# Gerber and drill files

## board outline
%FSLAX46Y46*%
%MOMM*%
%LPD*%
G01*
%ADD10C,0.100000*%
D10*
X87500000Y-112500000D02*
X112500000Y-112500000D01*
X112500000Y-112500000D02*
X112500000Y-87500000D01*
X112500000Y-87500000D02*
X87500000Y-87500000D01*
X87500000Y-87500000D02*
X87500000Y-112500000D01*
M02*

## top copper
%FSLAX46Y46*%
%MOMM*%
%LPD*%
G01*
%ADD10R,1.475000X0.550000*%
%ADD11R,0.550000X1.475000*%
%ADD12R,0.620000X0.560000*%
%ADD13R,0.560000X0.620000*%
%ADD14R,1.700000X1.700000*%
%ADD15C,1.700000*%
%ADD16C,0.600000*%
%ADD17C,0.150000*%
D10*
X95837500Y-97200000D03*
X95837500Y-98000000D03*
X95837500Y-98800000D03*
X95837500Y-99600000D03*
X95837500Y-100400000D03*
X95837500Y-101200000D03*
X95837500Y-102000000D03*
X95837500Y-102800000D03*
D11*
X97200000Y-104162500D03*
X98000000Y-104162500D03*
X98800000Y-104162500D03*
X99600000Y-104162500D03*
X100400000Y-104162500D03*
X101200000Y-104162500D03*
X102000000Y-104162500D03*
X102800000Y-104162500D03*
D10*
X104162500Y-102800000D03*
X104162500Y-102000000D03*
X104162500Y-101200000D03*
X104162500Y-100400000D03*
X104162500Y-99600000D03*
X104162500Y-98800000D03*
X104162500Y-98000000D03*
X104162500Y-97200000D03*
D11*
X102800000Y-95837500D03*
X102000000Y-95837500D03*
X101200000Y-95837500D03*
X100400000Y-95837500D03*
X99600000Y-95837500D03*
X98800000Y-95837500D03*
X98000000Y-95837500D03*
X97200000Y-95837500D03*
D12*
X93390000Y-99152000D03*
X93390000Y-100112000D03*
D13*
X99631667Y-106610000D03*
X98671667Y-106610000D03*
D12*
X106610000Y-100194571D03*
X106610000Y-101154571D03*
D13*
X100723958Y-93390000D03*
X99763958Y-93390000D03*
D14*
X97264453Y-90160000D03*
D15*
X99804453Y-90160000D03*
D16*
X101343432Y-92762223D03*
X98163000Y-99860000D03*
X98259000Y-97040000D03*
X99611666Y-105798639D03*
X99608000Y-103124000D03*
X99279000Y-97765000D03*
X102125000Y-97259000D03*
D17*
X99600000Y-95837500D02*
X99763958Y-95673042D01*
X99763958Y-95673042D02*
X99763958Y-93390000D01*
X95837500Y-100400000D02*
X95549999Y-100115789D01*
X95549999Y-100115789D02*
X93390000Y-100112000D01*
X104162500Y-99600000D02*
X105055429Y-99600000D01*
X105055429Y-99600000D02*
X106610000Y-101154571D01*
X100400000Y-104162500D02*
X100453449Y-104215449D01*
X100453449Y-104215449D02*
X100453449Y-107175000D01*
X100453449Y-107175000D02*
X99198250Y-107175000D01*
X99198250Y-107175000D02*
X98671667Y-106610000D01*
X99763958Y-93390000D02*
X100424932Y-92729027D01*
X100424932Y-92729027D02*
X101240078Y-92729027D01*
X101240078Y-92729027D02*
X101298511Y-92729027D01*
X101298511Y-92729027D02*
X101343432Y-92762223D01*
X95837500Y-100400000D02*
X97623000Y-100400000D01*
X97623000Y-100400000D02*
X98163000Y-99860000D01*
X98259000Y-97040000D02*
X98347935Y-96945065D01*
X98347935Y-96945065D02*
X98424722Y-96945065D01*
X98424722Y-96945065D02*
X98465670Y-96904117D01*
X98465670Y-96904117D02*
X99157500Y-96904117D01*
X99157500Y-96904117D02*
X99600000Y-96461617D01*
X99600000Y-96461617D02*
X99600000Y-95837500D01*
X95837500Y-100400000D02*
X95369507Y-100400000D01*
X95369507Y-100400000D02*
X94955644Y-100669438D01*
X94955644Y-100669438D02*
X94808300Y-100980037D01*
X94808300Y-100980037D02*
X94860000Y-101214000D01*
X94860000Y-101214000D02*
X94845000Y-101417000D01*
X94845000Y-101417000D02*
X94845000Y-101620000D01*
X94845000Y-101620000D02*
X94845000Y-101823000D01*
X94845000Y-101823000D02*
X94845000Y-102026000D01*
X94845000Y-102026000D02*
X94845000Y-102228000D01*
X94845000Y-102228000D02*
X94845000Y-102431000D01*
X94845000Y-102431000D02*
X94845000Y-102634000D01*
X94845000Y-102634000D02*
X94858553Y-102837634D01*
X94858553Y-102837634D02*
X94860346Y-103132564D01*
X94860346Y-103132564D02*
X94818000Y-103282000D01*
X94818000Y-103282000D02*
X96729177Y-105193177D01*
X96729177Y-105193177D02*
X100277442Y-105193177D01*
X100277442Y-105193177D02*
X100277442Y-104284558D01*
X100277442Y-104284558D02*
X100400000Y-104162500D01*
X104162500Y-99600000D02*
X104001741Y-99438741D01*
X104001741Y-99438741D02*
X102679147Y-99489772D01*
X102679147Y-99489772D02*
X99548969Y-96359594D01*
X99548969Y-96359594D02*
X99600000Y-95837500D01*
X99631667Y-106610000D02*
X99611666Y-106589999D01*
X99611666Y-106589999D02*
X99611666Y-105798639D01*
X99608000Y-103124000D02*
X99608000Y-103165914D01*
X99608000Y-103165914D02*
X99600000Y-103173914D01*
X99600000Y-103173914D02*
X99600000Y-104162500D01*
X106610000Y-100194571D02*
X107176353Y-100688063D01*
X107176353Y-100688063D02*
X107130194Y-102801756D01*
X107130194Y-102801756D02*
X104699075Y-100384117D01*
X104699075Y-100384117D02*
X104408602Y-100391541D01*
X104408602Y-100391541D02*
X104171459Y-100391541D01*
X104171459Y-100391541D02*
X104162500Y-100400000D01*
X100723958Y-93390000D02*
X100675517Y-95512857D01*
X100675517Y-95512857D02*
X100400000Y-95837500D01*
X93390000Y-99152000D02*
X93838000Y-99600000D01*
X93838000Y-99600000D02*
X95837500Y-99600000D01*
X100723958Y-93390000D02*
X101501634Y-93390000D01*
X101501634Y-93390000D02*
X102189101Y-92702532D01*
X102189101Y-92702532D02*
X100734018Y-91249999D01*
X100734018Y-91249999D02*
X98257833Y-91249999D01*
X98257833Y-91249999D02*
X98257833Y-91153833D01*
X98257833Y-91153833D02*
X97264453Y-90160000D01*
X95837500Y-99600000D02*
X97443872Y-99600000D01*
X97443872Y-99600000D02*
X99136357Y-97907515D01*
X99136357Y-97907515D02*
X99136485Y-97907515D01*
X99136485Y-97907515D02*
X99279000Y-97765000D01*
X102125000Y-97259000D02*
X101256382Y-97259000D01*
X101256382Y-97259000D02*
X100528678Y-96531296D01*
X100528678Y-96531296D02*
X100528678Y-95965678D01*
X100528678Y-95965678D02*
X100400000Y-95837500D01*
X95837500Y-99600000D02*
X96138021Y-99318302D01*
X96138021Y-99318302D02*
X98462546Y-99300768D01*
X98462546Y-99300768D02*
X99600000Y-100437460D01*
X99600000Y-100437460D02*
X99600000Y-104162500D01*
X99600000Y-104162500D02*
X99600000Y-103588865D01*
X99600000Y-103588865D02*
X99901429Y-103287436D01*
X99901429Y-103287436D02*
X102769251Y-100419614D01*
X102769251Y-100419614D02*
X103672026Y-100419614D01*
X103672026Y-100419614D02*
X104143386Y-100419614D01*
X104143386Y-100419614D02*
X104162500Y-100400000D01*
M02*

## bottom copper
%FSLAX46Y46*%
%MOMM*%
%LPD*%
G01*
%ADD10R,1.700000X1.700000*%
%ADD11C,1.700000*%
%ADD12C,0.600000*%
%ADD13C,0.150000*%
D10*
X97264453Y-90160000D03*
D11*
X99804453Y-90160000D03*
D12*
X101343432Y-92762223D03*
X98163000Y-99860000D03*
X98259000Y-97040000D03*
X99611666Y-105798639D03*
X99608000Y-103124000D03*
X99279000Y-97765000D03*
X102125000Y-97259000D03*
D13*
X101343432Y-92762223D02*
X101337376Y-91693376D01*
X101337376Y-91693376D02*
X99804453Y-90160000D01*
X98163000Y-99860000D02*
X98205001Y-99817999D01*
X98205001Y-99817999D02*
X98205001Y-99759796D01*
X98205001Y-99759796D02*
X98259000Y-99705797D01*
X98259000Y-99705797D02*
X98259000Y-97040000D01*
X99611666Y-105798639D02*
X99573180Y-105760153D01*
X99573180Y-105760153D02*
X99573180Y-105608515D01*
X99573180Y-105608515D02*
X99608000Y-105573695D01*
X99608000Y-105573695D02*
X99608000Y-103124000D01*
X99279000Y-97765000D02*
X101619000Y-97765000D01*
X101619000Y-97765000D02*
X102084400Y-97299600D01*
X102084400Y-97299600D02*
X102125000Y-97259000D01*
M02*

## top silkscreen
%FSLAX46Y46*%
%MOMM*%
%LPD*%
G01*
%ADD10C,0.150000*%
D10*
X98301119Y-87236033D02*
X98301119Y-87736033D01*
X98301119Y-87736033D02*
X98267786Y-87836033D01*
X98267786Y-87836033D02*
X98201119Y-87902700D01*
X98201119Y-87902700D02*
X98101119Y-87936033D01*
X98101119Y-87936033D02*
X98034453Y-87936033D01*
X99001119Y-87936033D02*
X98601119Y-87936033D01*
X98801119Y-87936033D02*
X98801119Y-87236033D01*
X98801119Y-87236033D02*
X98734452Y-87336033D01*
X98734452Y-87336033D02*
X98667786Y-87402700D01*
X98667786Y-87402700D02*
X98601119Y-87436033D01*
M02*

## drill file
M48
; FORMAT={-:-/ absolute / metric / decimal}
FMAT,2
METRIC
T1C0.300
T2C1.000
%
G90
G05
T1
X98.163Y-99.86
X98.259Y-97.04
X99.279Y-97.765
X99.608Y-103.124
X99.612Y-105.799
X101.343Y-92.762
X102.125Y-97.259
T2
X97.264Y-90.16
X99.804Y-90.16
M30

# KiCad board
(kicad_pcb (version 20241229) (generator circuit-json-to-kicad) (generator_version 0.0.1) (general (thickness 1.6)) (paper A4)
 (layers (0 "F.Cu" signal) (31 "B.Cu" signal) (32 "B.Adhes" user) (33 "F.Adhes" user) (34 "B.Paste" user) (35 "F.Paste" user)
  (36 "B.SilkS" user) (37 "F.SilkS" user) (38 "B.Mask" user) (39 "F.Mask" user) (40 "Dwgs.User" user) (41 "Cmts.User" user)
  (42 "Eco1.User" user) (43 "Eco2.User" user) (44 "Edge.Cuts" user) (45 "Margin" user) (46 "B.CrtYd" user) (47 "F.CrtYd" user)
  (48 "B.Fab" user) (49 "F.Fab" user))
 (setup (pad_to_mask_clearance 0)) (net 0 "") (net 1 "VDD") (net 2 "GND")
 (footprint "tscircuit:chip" (layer F.Cu) (at 100 100 0)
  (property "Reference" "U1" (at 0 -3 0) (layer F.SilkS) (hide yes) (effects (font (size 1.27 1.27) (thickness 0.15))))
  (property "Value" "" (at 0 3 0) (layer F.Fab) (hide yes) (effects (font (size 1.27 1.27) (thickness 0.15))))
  (pad "1" smd rect (at -4.1625 -2.8 0) (size 1.475 0.55) (layers F.Cu F.Mask))
  (pad "2" smd rect (at -4.1625 -2 0) (size 1.475 0.55) (layers F.Cu F.Mask))
  (pad "3" smd rect (at -4.1625 -1.2 0) (size 1.475 0.55) (layers F.Cu F.Mask))
  (pad "4" smd rect (at -4.1625 -0.4 0) (size 1.475 0.55) (layers F.Cu F.Mask) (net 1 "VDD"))
  (pad "5" smd rect (at -4.1625 0.4 0) (size 1.475 0.55) (layers F.Cu F.Mask) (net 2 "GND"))
  (pad "6" smd rect (at -4.1625 1.2 0) (size 1.475 0.55) (layers F.Cu F.Mask))
  (pad "7" smd rect (at -4.1625 2 0) (size 1.475 0.55) (layers F.Cu F.Mask))
  (pad "8" smd rect (at -4.1625 2.8 0) (size 1.475 0.55) (layers F.Cu F.Mask))
  (pad "9" smd rect (at -2.8 4.1625 0) (size 0.55 1.475) (layers F.Cu F.Mask))
  (pad "10" smd rect (at -2 4.1625 0) (size 0.55 1.475) (layers F.Cu F.Mask))
  (pad "11" smd rect (at -1.2 4.1625 0) (size 0.55 1.475) (layers F.Cu F.Mask))
  (pad "12" smd rect (at -0.4 4.1625 0) (size 0.55 1.475) (layers F.Cu F.Mask) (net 1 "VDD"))
  (pad "13" smd rect (at 0.4 4.1625 0) (size 0.55 1.475) (layers F.Cu F.Mask) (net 2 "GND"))
  (pad "14" smd rect (at 1.2 4.1625 0) (size 0.55 1.475) (layers F.Cu F.Mask))
  (pad "15" smd rect (at 2 4.1625 0) (size 0.55 1.475) (layers F.Cu F.Mask))
  (pad "16" smd rect (at 2.8 4.1625 0) (size 0.55 1.475) (layers F.Cu F.Mask))
  (pad "17" smd rect (at 4.1625 2.8 0) (size 1.475 0.55) (layers F.Cu F.Mask))
  (pad "18" smd rect (at 4.1625 2 0) (size 1.475 0.55) (layers F.Cu F.Mask))
  (pad "19" smd rect (at 4.1625 1.2 0) (size 1.475 0.55) (layers F.Cu F.Mask))
  (pad "20" smd rect (at 4.1625 0.4 0) (size 1.475 0.55) (layers F.Cu F.Mask) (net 1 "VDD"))
  (pad "21" smd rect (at 4.1625 -0.4 0) (size 1.475 0.55) (layers F.Cu F.Mask) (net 2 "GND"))
  (pad "22" smd rect (at 4.1625 -1.2 0) (size 1.475 0.55) (layers F.Cu F.Mask))
  (pad "23" smd rect (at 4.1625 -2 0) (size 1.475 0.55) (layers F.Cu F.Mask))
  (pad "24" smd rect (at 4.1625 -2.8 0) (size 1.475 0.55) (layers F.Cu F.Mask))
  (pad "25" smd rect (at 2.8 -4.1625 0) (size 0.55 1.475) (layers F.Cu F.Mask))
  (pad "26" smd rect (at 2 -4.1625 0) (size 0.55 1.475) (layers F.Cu F.Mask))
  (pad "27" smd rect (at 1.2 -4.1625 0) (size 0.55 1.475) (layers F.Cu F.Mask))
  (pad "28" smd rect (at 0.4 -4.1625 0) (size 0.55 1.475) (layers F.Cu F.Mask) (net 1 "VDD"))
  (pad "29" smd rect (at -0.4 -4.1625 0) (size 0.55 1.475) (layers F.Cu F.Mask) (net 2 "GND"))
  (pad "30" smd rect (at -1.2 -4.1625 0) (size 0.55 1.475) (layers F.Cu F.Mask))
  (pad "31" smd rect (at -2 -4.1625 0) (size 0.55 1.475) (layers F.Cu F.Mask))
  (pad "32" smd rect (at -2.8 -4.1625 0) (size 0.55 1.475) (layers F.Cu F.Mask))
  (pad "" smd rect (at -4.1625 -2.8 0) (size 1.0325 0.385) (layers F.Paste))
  (pad "" smd rect (at -4.1625 -2 0) (size 1.0325 0.385) (layers F.Paste))
  (pad "" smd rect (at -4.1625 -1.2 0) (size 1.0325 0.385) (layers F.Paste))
  (pad "" smd rect (at -4.1625 -0.4 0) (size 1.0325 0.385) (layers F.Paste))
  (pad "" smd rect (at -4.1625 0.4 0) (size 1.0325 0.385) (layers F.Paste))
  (pad "" smd rect (at -4.1625 1.2 0) (size 1.0325 0.385) (layers F.Paste))
  (pad "" smd rect (at -4.1625 2 0) (size 1.0325 0.385) (layers F.Paste))
  (pad "" smd rect (at -4.1625 2.8 0) (size 1.0325 0.385) (layers F.Paste))
  (pad "" smd rect (at -2.8 4.1625 0) (size 0.385 1.0325) (layers F.Paste))
  (pad "" smd rect (at -2 4.1625 0) (size 0.385 1.0325) (layers F.Paste))
  (pad "" smd rect (at -1.2 4.1625 0) (size 0.385 1.0325) (layers F.Paste))
  (pad "" smd rect (at -0.4 4.1625 0) (size 0.385 1.0325) (layers F.Paste))
  (pad "" smd rect (at 0.4 4.1625 0) (size 0.385 1.0325) (layers F.Paste))
  (pad "" smd rect (at 1.2 4.1625 0) (size 0.385 1.0325) (layers F.Paste))
  (pad "" smd rect (at 2 4.1625 0) (size 0.385 1.0325) (layers F.Paste))
  (pad "" smd rect (at 2.8 4.1625 0) (size 0.385 1.0325) (layers F.Paste))
  (pad "" smd rect (at 4.1625 2.8 0) (size 1.0325 0.385) (layers F.Paste))
  (pad "" smd rect (at 4.1625 2 0) (size 1.0325 0.385) (layers F.Paste))
  (pad "" smd rect (at 4.1625 1.2 0) (size 1.0325 0.385) (layers F.Paste))
  (pad "" smd rect (at 4.1625 0.4 0) (size 1.0325 0.385) (layers F.Paste))
  (pad "" smd rect (at 4.1625 -0.4 0) (size 1.0325 0.385) (layers F.Paste))
  (pad "" smd rect (at 4.1625 -1.2 0) (size 1.0325 0.385) (layers F.Paste))
  (pad "" smd rect (at 4.1625 -2 0) (size 1.0325 0.385) (layers F.Paste))
  (pad "" smd rect (at 4.1625 -2.8 0) (size 1.0325 0.385) (layers F.Paste))
  (pad "" smd rect (at 2.8 -4.1625 0) (size 0.385 1.0325) (layers F.Paste))
  (pad "" smd rect (at 2 -4.1625 0) (size 0.385 1.0325) (layers F.Paste))
  (pad "" smd rect (at 1.2 -4.1625 0) (size 0.385 1.0325) (layers F.Paste))
  (pad "" smd rect (at 0.4 -4.1625 0) (size 0.385 1.0325) (layers F.Paste))
  (pad "" smd rect (at -0.4 -4.1625 0) (size 0.385 1.0325) (layers F.Paste))
  (pad "" smd rect (at -1.2 -4.1625 0) (size 0.385 1.0325) (layers F.Paste))
  (pad "" smd rect (at -2 -4.1625 0) (size 0.385 1.0325) (layers F.Paste))
  (pad "" smd rect (at -2.8 -4.1625 0) (size 0.385 1.0325) (layers F.Paste)))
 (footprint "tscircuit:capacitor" (layer F.Cu) (at 93.39 99.632 -90.00000000000001)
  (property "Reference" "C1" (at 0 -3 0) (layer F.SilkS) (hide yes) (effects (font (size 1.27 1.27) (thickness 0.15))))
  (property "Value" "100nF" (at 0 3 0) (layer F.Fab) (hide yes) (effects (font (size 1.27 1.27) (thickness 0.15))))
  (pad "1" smd rect (at -0.48 0 0) (size 0.62 0.56) (layers F.Cu F.Mask) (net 1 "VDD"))
  (pad "2" smd rect (at 0.48 0 0) (size 0.62 0.56) (layers F.Cu F.Mask) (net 2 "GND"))
  (pad "" smd rect (at -0.48 0 0) (size 0.434 0.392) (layers F.Paste))
  (pad "" smd rect (at 0.48 0 0) (size 0.434 0.392) (layers F.Paste)))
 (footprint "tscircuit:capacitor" (layer F.Cu) (at 99.15166666666667 106.61 180)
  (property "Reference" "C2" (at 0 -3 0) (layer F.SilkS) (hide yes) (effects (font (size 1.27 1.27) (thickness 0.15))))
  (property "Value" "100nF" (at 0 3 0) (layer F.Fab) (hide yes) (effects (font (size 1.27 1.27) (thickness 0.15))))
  (pad "1" smd rect (at -0.48000000000000004 0 0) (size 0.56 0.62) (layers F.Cu F.Mask) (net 1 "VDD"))
  (pad "2" smd rect (at 0.47999999999999987 0 0) (size 0.56 0.62) (layers F.Cu F.Mask) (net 2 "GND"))
  (pad "" smd rect (at -0.48000000000000004 0 0) (size 0.392 0.434) (layers F.Paste))
  (pad "" smd rect (at 0.47999999999999987 0 0) (size 0.392 0.434) (layers F.Paste)))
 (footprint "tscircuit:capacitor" (layer F.Cu) (at 106.61 100.67457142857143 -90.00000000000001)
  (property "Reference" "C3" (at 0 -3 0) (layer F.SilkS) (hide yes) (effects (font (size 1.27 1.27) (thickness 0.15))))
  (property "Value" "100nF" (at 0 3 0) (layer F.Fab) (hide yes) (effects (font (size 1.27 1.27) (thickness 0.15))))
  (pad "1" smd rect (at -0.48 0 0) (size 0.62 0.56) (layers F.Cu F.Mask) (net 1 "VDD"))
  (pad "2" smd rect (at 0.4800000000000001 0 0) (size 0.62 0.56) (layers F.Cu F.Mask) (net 2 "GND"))
  (pad "" smd rect (at -0.48 0 0) (size 0.434 0.392) (layers F.Paste))
  (pad "" smd rect (at 0.4800000000000001 0 0) (size 0.434 0.392) (layers F.Paste)))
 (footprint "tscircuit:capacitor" (layer F.Cu) (at 100.24395833333334 93.39 180)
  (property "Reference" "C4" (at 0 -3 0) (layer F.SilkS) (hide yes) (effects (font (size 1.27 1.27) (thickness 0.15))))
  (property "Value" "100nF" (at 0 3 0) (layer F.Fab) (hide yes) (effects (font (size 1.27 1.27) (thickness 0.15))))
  (pad "1" smd rect (at -0.48 0 0) (size 0.56 0.62) (layers F.Cu F.Mask) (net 1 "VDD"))
  (pad "2" smd rect (at 0.48 0 0) (size 0.56 0.62) (layers F.Cu F.Mask) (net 2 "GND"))
  (pad "" smd rect (at -0.48 0 0) (size 0.392 0.434) (layers F.Paste))
  (pad "" smd rect (at 0.48 0 0) (size 0.392 0.434) (layers F.Paste)))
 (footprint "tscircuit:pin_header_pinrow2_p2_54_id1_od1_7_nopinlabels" (layer F.Cu) (at 98.534453125 90.16 0)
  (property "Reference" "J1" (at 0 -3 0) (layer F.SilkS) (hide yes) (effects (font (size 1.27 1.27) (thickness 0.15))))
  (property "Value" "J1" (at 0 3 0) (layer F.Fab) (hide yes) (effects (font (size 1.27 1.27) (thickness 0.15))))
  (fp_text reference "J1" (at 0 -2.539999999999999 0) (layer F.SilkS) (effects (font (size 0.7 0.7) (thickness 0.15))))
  (pad "1" thru_hole rect (at -1.27 0 0) (size 1.7 1.7) (drill 1) (layers *.Cu *.Mask) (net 1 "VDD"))
  (pad "2" thru_hole circle (at 1.27 0 0) (size 1.7 1.7) (drill 1) (layers *.Cu *.Mask) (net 2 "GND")))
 (segment (start 99.6 95.8375) (end 99.76395833333333 95.67304166666666) (width 0.15) (layer F.Cu) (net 2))
 (segment (start 99.76395833333333 95.67304166666666) (end 99.76395833333333 93.39) (width 0.15) (layer F.Cu) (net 2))
 (segment (start 95.8375 100.4) (end 95.54999882570709 100.11578913637184) (width 0.15) (layer F.Cu) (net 2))
 (segment (start 95.54999882570709 100.11578913637184) (end 93.39 100.112) (width 0.15) (layer F.Cu) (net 2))
 (segment (start 104.1625 99.6) (end 105.05542857142856 99.6) (width 0.15) (layer F.Cu) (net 2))
 (segment (start 105.05542857142856 99.6) (end 106.61 101.15457142857143) (width 0.15) (layer F.Cu) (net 2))
 (segment (start 100.4 104.1625) (end 100.45344876131234 104.21544876131235) (width 0.15) (layer F.Cu) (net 2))
 (segment (start 100.45344876131234 104.21544876131235) (end 100.45344876131234 107.175) (width 0.15) (layer F.Cu) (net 2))
 (segment (start 100.45344876131234 107.175) (end 99.19824993292859 107.175) (width 0.15) (layer F.Cu) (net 2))
 (segment (start 99.19824993292859 107.175) (end 98.67166666666667 106.61) (width 0.15) (layer F.Cu) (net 2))
 (segment (start 99.76395833333333 93.39) (end 100.42493155843435 92.72902677489898) (width 0.15) (layer F.Cu) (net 2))
 (segment (start 100.42493155843435 92.72902677489898) (end 101.24007779189273 92.72902677489898) (width 0.15) (layer F.Cu) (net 2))
 (segment (start 101.24007779189273 92.72902677489898) (end 101.2985105056803 92.72902677489898) (width 0.15) (layer F.Cu) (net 2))
 (segment (start 101.2985105056803 92.72902677489898) (end 101.34343219516313 92.76222256666912) (width 0.15) (layer F.Cu) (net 2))
 (segment (start 101.34343219516313 92.76222256666912) (end 101.33737570534065 91.69337570534066) (width 0.15) (layer B.Cu) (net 2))
 (segment (start 101.33737570534065 91.69337570534066) (end 99.804453125 90.16) (width 0.15) (layer B.Cu) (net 2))
 (segment (start 95.8375 100.4) (end 97.623 100.4) (width 0.15) (layer F.Cu) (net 2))
 (segment (start 97.623 100.4) (end 98.163 99.86) (width 0.15) (layer F.Cu) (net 2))
 (segment (start 98.163 99.86) (end 98.20500076413374 99.81799923586625) (width 0.15) (layer B.Cu) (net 2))
 (segment (start 98.20500076413374 99.81799923586625) (end 98.20500076413374 99.75979623298763) (width 0.15) (layer B.Cu) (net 2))
 (segment (start 98.20500076413374 99.75979623298763) (end 98.259 99.70579699712138) (width 0.15) (layer B.Cu) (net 2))
 (segment (start 98.259 99.70579699712138) (end 98.259 97.04) (width 0.15) (layer B.Cu) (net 2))
 (segment (start 98.259 97.04) (end 98.34793469358411 96.9450653064159) (width 0.15) (layer F.Cu) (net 2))
 (segment (start 98.34793469358411 96.9450653064159) (end 98.4247223865256 96.9450653064159) (width 0.15) (layer F.Cu) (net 2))
 (segment (start 98.4247223865256 96.9450653064159) (end 98.46567033995531 96.90411735298619) (width 0.15) (layer F.Cu) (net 2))
 (segment (start 98.46567033995531 96.90411735298619) (end 99.15749956172179 96.90411735298619) (width 0.15) (layer F.Cu) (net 2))
 (segment (start 99.15749956172179 96.90411735298619) (end 99.6 96.46161691470799) (width 0.15) (layer F.Cu) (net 2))
 (segment (start 99.6 96.46161691470799) (end 99.6 95.8375) (width 0.15) (layer F.Cu) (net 2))
 (segment (start 95.8375 100.4) (end 95.36950657616131 100.4) (width 0.15) (layer F.Cu) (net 2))
 (segment (start 95.36950657616131 100.4) (end 94.95564404651859 100.66943775485414) (width 0.15) (layer F.Cu) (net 2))
 (segment (start 94.95564404651859 100.66943775485414) (end 94.80829993462471 100.98003654561826) (width 0.15) (layer F.Cu) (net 2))
 (segment (start 94.80829993462471 100.98003654561826) (end 94.86 101.214) (width 0.15) (layer F.Cu) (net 2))
 (segment (start 94.86 101.214) (end 94.845 101.417) (width 0.15) (layer F.Cu) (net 2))
 (segment (start 94.845 101.417) (end 94.845 101.62) (width 0.15) (layer F.Cu) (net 2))
 (segment (start 94.845 101.62) (end 94.845 101.823) (width 0.15) (layer F.Cu) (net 2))
 (segment (start 94.845 101.823) (end 94.845 102.026) (width 0.15) (layer F.Cu) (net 2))
 (segment (start 94.845 102.026) (end 94.845 102.228) (width 0.15) (layer F.Cu) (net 2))
 (segment (start 94.845 102.228) (end 94.845 102.431) (width 0.15) (layer F.Cu) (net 2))
 (segment (start 94.845 102.431) (end 94.845 102.634) (width 0.15) (layer F.Cu) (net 2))
 (segment (start 94.845 102.634) (end 94.85855329042725 102.83763390606946) (width 0.15) (layer F.Cu) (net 2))
 (segment (start 94.85855329042725 102.83763390606946) (end 94.86034600494294 103.1325643967498) (width 0.15) (layer F.Cu) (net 2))
 (segment (start 94.86034600494294 103.1325643967498) (end 94.818 103.282) (width 0.15) (layer F.Cu) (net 2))
 (segment (start 94.818 103.282) (end 96.72917663282733 105.19317663282735) (width 0.15) (layer F.Cu) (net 2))
 (segment (start 96.72917663282733 105.19317663282735) (end 100.27744164139212 105.19317663282735) (width 0.15) (layer F.Cu) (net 2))
 (segment (start 100.27744164139212 105.19317663282735) (end 100.27744164139212 104.28455835860788) (width 0.15) (layer F.Cu) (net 2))
 (segment (start 100.27744164139212 104.28455835860788) (end 100.4 104.1625) (width 0.15) (layer F.Cu) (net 2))
 (segment (start 104.1625 99.6) (end 104.00174073680326 99.43874073680325) (width 0.15) (layer F.Cu) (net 2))
 (segment (start 104.00174073680326 99.43874073680325) (end 102.67914711390605 99.4897715723112) (width 0.15) (layer F.Cu) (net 2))
 (segment (start 102.67914711390605 99.4897715723112) (end 99.54896916449205 96.3595936228972) (width 0.15) (layer F.Cu) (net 2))
 (segment (start 99.54896916449205 96.3595936228972) (end 99.6 95.8375) (width 0.15) (layer F.Cu) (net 2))
 (segment (start 99.63166666666666 106.61) (end 99.61166566666667 106.589999) (width 0.15) (layer F.Cu) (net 1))
 (segment (start 99.61166566666667 106.589999) (end 99.61166566666667 105.79863874701397) (width 0.15) (layer F.Cu) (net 1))
 (segment (start 99.61166566666667 105.79863874701397) (end 99.57318040827276 105.76015348862006) (width 0.15) (layer B.Cu) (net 1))
 (segment (start 99.57318040827276 105.76015348862006) (end 99.57318040827276 105.60851499635852) (width 0.15) (layer B.Cu) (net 1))
 (segment (start 99.57318040827276 105.60851499635852) (end 99.608 105.5736954046313) (width 0.15) (layer B.Cu) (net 1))
 (segment (start 99.608 105.5736954046313) (end 99.608 103.124) (width 0.15) (layer B.Cu) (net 1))
 (segment (start 99.608 103.124) (end 99.608 103.1659144450318) (width 0.15) (layer F.Cu) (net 1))
 (segment (start 99.608 103.1659144450318) (end 99.6 103.1739144450318) (width 0.15) (layer F.Cu) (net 1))
 (segment (start 99.6 103.1739144450318) (end 99.6 104.1625) (width 0.15) (layer F.Cu) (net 1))
 (segment (start 106.61 100.19457142857144) (end 107.17635324123205 100.68806333603553) (width 0.15) (layer F.Cu) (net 1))
 (segment (start 107.17635324123205 100.68806333603553) (end 107.13019352955445 102.80175552600008) (width 0.15) (layer F.Cu) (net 1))
 (segment (start 107.13019352955445 102.80175552600008) (end 104.69907519326506 100.3841168898164) (width 0.15) (layer F.Cu) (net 1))
 (segment (start 104.69907519326506 100.3841168898164) (end 104.40860228240784 100.39154060927434) (width 0.15) (layer F.Cu) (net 1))
 (segment (start 104.40860228240784 100.39154060927434) (end 104.17145939072566 100.39154060927434) (width 0.15) (layer F.Cu) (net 1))
 (segment (start 104.17145939072566 100.39154060927434) (end 104.1625 100.4) (width 0.15) (layer F.Cu) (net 1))
 (segment (start 100.72395833333333 93.39) (end 100.67551732443452 95.51285656429572) (width 0.15) (layer F.Cu) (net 1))
 (segment (start 100.67551732443452 95.51285656429572) (end 100.4 95.8375) (width 0.15) (layer F.Cu) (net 1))
 (segment (start 93.39 99.152) (end 93.838 99.6) (width 0.15) (layer F.Cu) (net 1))
 (segment (start 93.838 99.6) (end 95.8375 99.6) (width 0.15) (layer F.Cu) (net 1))
 (segment (start 100.72395833333333 93.39) (end 101.50163371453306 93.39) (width 0.15) (layer F.Cu) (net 1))
 (segment (start 101.50163371453306 93.39) (end 102.1891012837175 92.70253243081554) (width 0.15) (layer F.Cu) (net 1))
 (segment (start 102.1891012837175 92.70253243081554) (end 100.73401771236857 91.24999875432592) (width 0.15) (layer F.Cu) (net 1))
 (segment (start 100.73401771236857 91.24999875432592) (end 98.25783285511247 91.24999875432592) (width 0.15) (layer F.Cu) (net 1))
 (segment (start 98.25783285511247 91.24999875432592) (end 98.25783285511247 91.15383285511248) (width 0.15) (layer F.Cu) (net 1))
 (segment (start 98.25783285511247 91.15383285511248) (end 97.264453125 90.16) (width 0.15) (layer F.Cu) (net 1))
 (segment (start 95.8375 99.6) (end 97.4438721049453 99.6) (width 0.15) (layer F.Cu) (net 1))
 (segment (start 97.4438721049453 99.6) (end 99.13635711153833 97.90751499340698) (width 0.15) (layer F.Cu) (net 1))
 (segment (start 99.13635711153833 97.90751499340698) (end 99.13648500659302 97.90751499340698) (width 0.15) (layer F.Cu) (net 1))
 (segment (start 99.13648500659302 97.90751499340698) (end 99.279 97.765) (width 0.15) (layer F.Cu) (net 1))
 (segment (start 99.279 97.765) (end 101.619 97.765) (width 0.15) (layer B.Cu) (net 1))
 (segment (start 101.619 97.765) (end 102.08439989215097 97.29960010784902) (width 0.15) (layer B.Cu) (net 1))
 (segment (start 102.08439989215097 97.29960010784902) (end 102.125 97.259) (width 0.15) (layer B.Cu) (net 1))
 (segment (start 102.125 97.259) (end 101.25638237039455 97.259) (width 0.15) (layer F.Cu) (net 1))
 (segment (start 101.25638237039455 97.259) (end 100.52867808884149 96.53129571844694) (width 0.15) (layer F.Cu) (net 1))
 (segment (start 100.52867808884149 96.53129571844694) (end 100.52867808884149 95.96567808884149) (width 0.15) (layer F.Cu) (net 1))
 (segment (start 100.52867808884149 95.96567808884149) (end 100.4 95.8375) (width 0.15) (layer F.Cu) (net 1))
 (segment (start 95.8375 99.6) (end 96.13802115011137 99.31830211046508) (width 0.15) (layer F.Cu) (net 1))
 (segment (start 96.13802115011137 99.31830211046508) (end 98.4625463687967 99.30076849192618) (width 0.15) (layer F.Cu) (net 1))
 (segment (start 98.4625463687967 99.30076849192618) (end 99.6 100.43745977914735) (width 0.15) (layer F.Cu) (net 1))
 (segment (start 99.6 100.43745977914735) (end 99.6 104.1625) (width 0.15) (layer F.Cu) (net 1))
 (segment (start 99.6 104.1625) (end 99.6 103.58886460672694) (width 0.15) (layer F.Cu) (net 1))
 (segment (start 99.6 103.58886460672694) (end 99.90142905857718 103.28743554814977) (width 0.15) (layer F.Cu) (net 1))
 (segment (start 99.90142905857718 103.28743554814977) (end 102.76925060355296 100.41961400317399) (width 0.15) (layer F.Cu) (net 1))
 (segment (start 102.76925060355296 100.41961400317399) (end 103.6720264802097 100.41961400317399) (width 0.15) (layer F.Cu) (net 1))
 (segment (start 103.6720264802097 100.41961400317399) (end 104.14338599682601 100.41961400317399) (width 0.15) (layer F.Cu) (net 1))
 (segment (start 104.14338599682601 100.41961400317399) (end 104.1625 100.4) (width 0.15) (layer F.Cu) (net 1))
 (gr_line (start 87.5 112.5) (end 112.5 112.5) (width 0.1) (layer Edge.Cuts))
 (gr_line (start 112.5 112.5) (end 112.5 87.5) (width 0.1) (layer Edge.Cuts))
 (gr_line (start 112.5 87.5) (end 87.5 87.5) (width 0.1) (layer Edge.Cuts))
 (gr_line (start 87.5 87.5) (end 87.5 112.5) (width 0.1) (layer Edge.Cuts))
 (via (at 101.34343219516313 92.76222256666912) (size 0.6) (drill 0.3) (layers F.Cu B.Cu) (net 2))
 (via (at 98.163 99.86) (size 0.6) (drill 0.3) (layers F.Cu B.Cu) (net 2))
 (via (at 98.259 97.04) (size 0.6) (drill 0.3) (layers F.Cu B.Cu) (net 2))
 (via (at 99.61166566666667 105.79863874701397) (size 0.6) (drill 0.3) (layers F.Cu B.Cu) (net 1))
 (via (at 99.608 103.124) (size 0.6) (drill 0.3) (layers F.Cu B.Cu) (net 1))
 (via (at 99.279 97.765) (size 0.6) (drill 0.3) (layers F.Cu B.Cu) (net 1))
 (via (at 102.125 97.259) (size 0.6) (drill 0.3) (layers F.Cu B.Cu) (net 1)))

